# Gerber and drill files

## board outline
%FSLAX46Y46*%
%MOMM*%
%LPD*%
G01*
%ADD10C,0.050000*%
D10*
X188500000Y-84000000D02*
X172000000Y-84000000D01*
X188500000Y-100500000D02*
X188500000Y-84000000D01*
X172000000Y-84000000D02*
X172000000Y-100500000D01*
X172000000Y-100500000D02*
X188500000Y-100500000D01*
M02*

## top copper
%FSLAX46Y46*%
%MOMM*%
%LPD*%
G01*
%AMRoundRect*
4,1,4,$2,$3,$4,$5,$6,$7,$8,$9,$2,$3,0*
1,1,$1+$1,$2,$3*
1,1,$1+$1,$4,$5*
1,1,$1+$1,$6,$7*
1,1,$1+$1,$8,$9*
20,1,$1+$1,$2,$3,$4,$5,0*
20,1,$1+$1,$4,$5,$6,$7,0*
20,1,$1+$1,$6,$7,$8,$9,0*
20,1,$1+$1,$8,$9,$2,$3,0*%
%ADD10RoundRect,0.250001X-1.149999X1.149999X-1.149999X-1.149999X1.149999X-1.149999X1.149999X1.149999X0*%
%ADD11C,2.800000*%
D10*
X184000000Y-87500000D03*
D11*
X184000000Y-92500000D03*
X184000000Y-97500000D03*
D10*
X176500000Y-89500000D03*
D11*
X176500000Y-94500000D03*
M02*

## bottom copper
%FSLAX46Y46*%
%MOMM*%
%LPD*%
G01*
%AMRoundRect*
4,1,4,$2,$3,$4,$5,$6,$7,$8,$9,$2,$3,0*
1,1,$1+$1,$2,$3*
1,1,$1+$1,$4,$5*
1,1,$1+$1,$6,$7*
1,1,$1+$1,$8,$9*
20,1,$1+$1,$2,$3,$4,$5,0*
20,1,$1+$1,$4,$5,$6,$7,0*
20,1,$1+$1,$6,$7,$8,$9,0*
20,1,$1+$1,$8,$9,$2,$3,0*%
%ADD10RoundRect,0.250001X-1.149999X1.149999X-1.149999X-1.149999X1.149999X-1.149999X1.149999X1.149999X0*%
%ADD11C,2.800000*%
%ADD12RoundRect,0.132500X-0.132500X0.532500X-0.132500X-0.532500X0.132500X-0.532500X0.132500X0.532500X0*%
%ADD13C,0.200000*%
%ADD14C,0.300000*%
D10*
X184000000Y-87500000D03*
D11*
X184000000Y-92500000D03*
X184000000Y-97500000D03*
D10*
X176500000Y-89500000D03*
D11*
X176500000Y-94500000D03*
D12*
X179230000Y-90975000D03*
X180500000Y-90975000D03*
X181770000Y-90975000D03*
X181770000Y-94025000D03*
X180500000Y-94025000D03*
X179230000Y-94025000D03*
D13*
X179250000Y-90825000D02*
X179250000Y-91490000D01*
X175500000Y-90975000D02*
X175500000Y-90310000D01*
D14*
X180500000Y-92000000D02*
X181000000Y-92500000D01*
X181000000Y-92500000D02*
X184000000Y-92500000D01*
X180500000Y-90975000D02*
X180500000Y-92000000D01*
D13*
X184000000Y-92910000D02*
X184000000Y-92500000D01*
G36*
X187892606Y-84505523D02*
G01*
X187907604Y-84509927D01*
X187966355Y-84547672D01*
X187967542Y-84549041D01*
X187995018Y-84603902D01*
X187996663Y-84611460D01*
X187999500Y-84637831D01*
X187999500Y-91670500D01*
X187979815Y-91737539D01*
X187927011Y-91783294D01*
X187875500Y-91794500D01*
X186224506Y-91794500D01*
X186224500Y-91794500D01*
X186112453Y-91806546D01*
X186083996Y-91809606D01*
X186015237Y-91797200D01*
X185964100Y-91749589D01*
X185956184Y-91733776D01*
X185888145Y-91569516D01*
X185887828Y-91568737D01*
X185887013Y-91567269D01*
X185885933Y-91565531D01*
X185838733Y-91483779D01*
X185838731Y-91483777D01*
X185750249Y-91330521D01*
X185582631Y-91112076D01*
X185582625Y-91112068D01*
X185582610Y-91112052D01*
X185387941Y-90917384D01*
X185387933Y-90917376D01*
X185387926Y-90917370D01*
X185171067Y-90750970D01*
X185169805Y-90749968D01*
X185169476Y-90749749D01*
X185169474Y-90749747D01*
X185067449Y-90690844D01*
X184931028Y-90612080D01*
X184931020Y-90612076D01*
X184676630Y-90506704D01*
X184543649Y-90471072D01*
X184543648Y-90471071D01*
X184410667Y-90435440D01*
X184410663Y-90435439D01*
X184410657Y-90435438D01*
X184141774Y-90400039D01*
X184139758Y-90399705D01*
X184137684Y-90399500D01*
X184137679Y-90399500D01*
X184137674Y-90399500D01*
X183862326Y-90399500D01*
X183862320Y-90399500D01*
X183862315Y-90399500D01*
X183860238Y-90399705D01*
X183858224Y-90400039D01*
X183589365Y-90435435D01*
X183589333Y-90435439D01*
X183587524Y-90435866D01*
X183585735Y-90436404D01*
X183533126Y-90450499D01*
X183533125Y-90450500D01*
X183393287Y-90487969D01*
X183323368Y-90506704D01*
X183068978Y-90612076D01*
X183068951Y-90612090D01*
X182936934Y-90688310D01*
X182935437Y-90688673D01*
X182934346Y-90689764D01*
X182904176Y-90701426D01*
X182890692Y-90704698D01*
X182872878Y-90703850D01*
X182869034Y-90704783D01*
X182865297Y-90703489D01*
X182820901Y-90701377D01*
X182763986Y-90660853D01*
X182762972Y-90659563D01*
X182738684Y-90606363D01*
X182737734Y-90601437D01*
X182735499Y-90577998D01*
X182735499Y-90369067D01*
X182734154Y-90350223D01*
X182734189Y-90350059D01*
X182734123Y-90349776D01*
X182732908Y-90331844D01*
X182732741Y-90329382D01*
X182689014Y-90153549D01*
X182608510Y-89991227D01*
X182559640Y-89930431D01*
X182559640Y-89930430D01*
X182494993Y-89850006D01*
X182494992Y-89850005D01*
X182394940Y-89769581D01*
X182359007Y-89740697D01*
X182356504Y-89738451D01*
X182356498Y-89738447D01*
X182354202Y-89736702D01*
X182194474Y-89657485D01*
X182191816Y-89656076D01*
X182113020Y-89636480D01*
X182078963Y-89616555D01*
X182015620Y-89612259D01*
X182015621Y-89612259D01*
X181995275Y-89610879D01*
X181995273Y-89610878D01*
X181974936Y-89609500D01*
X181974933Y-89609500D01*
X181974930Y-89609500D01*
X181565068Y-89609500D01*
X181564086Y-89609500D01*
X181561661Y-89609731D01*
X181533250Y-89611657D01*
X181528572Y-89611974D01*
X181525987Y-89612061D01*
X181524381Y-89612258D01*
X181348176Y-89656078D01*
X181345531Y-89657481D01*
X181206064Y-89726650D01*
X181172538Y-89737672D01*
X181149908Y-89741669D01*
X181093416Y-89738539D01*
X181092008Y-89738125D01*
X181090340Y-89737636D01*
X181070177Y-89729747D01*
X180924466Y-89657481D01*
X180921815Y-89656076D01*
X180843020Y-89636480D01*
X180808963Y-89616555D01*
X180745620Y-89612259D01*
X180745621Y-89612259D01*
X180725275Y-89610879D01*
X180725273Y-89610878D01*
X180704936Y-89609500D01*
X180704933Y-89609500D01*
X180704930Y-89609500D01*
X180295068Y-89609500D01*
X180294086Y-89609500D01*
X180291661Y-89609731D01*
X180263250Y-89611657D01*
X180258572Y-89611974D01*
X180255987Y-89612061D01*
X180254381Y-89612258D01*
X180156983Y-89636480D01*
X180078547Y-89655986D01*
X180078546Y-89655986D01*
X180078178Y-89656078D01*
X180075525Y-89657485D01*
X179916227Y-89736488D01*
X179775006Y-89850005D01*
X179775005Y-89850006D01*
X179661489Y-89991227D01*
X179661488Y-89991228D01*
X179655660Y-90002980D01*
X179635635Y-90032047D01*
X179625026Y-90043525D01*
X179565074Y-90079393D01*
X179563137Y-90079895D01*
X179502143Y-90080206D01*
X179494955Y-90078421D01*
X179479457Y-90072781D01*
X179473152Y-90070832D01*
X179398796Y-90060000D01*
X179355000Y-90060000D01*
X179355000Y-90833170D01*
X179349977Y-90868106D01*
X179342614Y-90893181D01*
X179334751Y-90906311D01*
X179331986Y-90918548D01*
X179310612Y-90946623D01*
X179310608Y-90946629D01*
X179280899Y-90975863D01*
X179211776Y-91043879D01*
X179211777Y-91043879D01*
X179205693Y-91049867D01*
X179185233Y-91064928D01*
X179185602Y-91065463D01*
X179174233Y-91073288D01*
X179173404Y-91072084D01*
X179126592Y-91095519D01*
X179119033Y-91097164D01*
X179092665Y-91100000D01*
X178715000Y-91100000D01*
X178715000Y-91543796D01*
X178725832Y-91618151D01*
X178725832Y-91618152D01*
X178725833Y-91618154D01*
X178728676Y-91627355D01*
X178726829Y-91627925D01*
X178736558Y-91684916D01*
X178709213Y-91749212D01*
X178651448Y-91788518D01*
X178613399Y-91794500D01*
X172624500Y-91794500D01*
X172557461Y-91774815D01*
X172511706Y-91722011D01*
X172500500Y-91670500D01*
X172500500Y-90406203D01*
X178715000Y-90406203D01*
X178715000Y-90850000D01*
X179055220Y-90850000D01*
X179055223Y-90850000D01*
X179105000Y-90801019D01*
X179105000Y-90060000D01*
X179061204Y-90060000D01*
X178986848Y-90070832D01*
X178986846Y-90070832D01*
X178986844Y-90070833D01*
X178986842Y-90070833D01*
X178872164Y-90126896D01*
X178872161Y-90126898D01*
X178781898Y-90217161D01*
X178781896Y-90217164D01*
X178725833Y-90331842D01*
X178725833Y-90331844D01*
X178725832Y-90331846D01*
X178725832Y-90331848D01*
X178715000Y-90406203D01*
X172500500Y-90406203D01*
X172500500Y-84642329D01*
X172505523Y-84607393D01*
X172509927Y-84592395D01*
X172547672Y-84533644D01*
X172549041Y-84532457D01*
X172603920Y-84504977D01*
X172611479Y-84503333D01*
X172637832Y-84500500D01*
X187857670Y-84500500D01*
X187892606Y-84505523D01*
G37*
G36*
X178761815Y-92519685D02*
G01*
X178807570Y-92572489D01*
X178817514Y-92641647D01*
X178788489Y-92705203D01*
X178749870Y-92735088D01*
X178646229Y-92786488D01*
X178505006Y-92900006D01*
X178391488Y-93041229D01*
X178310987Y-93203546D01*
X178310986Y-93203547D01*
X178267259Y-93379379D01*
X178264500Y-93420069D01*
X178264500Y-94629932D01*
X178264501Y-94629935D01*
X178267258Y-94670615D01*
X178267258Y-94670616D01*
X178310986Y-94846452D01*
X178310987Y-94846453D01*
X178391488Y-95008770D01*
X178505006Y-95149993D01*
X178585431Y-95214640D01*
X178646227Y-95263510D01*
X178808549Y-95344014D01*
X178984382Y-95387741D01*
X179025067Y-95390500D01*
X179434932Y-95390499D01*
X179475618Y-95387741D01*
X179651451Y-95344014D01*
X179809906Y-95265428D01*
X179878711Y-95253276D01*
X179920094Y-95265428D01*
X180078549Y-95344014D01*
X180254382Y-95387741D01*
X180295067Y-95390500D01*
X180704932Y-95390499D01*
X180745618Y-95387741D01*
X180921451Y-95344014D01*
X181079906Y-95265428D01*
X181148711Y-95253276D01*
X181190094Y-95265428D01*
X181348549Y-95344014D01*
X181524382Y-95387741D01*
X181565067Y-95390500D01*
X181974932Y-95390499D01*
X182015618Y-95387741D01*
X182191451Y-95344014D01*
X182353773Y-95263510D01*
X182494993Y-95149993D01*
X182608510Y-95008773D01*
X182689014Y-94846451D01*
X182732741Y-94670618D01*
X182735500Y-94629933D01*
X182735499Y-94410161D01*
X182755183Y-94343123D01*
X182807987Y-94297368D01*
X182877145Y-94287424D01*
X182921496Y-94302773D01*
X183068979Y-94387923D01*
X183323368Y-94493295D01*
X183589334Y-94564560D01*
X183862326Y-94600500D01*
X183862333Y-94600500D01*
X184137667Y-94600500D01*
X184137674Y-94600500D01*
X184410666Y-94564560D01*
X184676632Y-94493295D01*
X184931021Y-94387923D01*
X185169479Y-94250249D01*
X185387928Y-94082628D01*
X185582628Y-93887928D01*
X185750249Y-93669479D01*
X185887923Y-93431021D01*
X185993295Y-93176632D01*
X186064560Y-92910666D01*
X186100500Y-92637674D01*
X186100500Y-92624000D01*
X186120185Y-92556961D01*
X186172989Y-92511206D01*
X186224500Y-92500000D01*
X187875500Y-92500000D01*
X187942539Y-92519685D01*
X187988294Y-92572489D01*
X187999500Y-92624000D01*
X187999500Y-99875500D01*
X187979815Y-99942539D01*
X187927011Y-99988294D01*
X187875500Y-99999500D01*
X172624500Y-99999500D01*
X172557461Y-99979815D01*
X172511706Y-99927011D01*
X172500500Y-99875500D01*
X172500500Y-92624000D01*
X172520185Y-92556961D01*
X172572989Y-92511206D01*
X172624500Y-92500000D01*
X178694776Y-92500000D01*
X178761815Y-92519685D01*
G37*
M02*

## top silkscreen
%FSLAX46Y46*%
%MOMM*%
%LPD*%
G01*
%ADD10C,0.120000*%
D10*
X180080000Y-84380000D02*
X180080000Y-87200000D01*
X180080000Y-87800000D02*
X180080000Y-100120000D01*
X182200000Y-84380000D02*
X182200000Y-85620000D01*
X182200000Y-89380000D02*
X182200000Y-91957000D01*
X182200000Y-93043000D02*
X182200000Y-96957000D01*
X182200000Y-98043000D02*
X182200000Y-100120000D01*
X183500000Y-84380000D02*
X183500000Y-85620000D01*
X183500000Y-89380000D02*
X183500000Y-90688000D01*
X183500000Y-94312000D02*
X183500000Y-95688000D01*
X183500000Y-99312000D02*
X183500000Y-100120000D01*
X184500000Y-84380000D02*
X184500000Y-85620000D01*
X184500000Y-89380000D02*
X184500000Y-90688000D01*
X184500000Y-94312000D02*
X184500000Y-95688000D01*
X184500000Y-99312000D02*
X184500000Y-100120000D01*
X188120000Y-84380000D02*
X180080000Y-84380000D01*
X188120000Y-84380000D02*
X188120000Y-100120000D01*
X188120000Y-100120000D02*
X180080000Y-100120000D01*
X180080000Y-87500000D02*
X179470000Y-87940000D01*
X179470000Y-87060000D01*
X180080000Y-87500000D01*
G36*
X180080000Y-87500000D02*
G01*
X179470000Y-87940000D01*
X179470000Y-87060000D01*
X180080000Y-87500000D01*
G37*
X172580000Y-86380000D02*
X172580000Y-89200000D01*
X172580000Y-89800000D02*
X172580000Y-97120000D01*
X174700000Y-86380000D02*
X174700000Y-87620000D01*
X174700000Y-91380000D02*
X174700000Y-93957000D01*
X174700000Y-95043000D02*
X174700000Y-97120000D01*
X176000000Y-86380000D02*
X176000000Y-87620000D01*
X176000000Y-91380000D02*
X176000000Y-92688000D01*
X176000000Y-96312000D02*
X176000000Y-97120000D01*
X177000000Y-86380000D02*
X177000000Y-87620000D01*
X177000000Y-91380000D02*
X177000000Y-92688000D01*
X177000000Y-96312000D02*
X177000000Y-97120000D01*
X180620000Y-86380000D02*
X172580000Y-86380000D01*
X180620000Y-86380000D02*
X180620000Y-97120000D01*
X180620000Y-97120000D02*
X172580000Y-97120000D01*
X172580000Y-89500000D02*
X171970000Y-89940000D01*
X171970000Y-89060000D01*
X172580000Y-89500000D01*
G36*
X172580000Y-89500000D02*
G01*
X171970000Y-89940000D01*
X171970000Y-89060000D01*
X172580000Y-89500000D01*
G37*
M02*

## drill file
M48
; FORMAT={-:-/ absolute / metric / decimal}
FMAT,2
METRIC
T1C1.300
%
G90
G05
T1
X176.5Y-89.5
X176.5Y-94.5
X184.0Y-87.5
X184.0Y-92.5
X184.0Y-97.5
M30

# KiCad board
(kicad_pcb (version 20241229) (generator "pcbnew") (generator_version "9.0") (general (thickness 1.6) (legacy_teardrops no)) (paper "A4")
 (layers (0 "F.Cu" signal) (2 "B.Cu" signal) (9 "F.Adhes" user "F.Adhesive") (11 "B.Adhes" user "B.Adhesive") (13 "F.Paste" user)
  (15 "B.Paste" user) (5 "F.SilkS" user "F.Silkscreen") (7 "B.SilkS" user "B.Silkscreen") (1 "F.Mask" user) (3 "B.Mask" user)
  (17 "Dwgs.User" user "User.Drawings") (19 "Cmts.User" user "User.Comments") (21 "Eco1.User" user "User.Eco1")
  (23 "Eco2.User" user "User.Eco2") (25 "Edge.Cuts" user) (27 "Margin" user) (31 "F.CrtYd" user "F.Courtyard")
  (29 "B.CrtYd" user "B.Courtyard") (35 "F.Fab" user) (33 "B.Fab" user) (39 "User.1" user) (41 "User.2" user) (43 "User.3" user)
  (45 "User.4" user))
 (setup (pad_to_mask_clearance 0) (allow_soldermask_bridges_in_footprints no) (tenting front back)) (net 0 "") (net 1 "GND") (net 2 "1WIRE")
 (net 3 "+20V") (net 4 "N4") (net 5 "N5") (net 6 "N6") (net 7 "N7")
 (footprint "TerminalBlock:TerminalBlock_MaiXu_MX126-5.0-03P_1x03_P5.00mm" (layer "F.Cu") (at 184 87.5 -90)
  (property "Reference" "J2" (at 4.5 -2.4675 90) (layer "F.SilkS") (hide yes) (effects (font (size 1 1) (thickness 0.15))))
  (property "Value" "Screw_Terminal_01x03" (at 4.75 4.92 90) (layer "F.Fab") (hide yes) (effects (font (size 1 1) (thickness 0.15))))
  (fp_line (start -3.12 3.92) (end -0.3 3.92) (stroke (width 0.12) (type solid)) (layer "F.SilkS"))
  (fp_line (start 0.3 3.92) (end 12.62 3.92) (stroke (width 0.12) (type solid)) (layer "F.SilkS"))
  (fp_line (start -3.12 1.8) (end -1.88 1.8) (stroke (width 0.12) (type solid)) (layer "F.SilkS"))
  (fp_line (start 1.88 1.8) (end 4.457 1.8) (stroke (width 0.12) (type solid)) (layer "F.SilkS"))
  (fp_line (start 5.543 1.8) (end 9.457 1.8) (stroke (width 0.12) (type solid)) (layer "F.SilkS"))
  (fp_line (start 10.543 1.8) (end 12.62 1.8) (stroke (width 0.12) (type solid)) (layer "F.SilkS"))
  (fp_line (start -3.12 0.5) (end -1.88 0.5) (stroke (width 0.12) (type solid)) (layer "F.SilkS"))
  (fp_line (start 1.88 0.5) (end 3.188 0.5) (stroke (width 0.12) (type solid)) (layer "F.SilkS"))
  (fp_line (start 6.812 0.5) (end 8.188 0.5) (stroke (width 0.12) (type solid)) (layer "F.SilkS"))
  (fp_line (start 11.812 0.5) (end 12.62 0.5) (stroke (width 0.12) (type solid)) (layer "F.SilkS"))
  (fp_line (start -3.12 -0.5) (end -1.88 -0.5) (stroke (width 0.12) (type solid)) (layer "F.SilkS"))
  (fp_line (start 1.88 -0.5) (end 3.188 -0.5) (stroke (width 0.12) (type solid)) (layer "F.SilkS"))
  (fp_line (start 6.812 -0.5) (end 8.188 -0.5) (stroke (width 0.12) (type solid)) (layer "F.SilkS"))
  (fp_line (start 11.812 -0.5) (end 12.62 -0.5) (stroke (width 0.12) (type solid)) (layer "F.SilkS"))
  (fp_line (start -3.12 -4.12) (end -3.12 3.92) (stroke (width 0.12) (type solid)) (layer "F.SilkS"))
  (fp_line (start -3.12 -4.12) (end 12.62 -4.12) (stroke (width 0.12) (type solid)) (layer "F.SilkS"))
  (fp_line (start 12.62 -4.12) (end 12.62 3.92) (stroke (width 0.12) (type solid)) (layer "F.SilkS"))
  (fp_poly (pts (xy 0 3.92) (xy 0.44 4.53) (xy -0.44 4.53)) (stroke (width 0.12) (type solid)) (fill yes) (layer "F.SilkS"))
  (pad "1" thru_hole roundrect (at 0 0 270) (size 2.8 2.8) (drill 1.3) (layers "*.Cu" "*.Mask") (remove_unused_layers no)
   (roundrect_rratio 0.089286) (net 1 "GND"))
  (pad "2" thru_hole circle (at 5 0 270) (size 2.8 2.8) (drill 1.3) (layers "*.Cu" "*.Mask") (remove_unused_layers no) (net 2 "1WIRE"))
  (pad "3" thru_hole circle (at 10 0 270) (size 2.8 2.8) (drill 1.3) (layers "*.Cu" "*.Mask") (remove_unused_layers no) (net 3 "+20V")))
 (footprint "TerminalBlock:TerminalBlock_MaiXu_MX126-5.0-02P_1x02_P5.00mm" (layer "F.Cu") (at 176.5 89.5 -90)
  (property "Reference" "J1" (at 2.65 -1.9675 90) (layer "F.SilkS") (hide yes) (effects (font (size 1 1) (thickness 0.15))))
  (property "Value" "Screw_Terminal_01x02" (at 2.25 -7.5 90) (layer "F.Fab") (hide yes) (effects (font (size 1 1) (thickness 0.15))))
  (fp_line (start -3.12 3.92) (end -0.3 3.92) (stroke (width 0.12) (type solid)) (layer "F.SilkS"))
  (fp_line (start 0.3 3.92) (end 7.62 3.92) (stroke (width 0.12) (type solid)) (layer "F.SilkS"))
  (fp_line (start -3.12 1.8) (end -1.88 1.8) (stroke (width 0.12) (type solid)) (layer "F.SilkS"))
  (fp_line (start 1.88 1.8) (end 4.457 1.8) (stroke (width 0.12) (type solid)) (layer "F.SilkS"))
  (fp_line (start 5.543 1.8) (end 7.62 1.8) (stroke (width 0.12) (type solid)) (layer "F.SilkS"))
  (fp_line (start -3.12 0.5) (end -1.88 0.5) (stroke (width 0.12) (type solid)) (layer "F.SilkS"))
  (fp_line (start 1.88 0.5) (end 3.188 0.5) (stroke (width 0.12) (type solid)) (layer "F.SilkS"))
  (fp_line (start 6.812 0.5) (end 7.62 0.5) (stroke (width 0.12) (type solid)) (layer "F.SilkS"))
  (fp_line (start -3.12 -0.5) (end -1.88 -0.5) (stroke (width 0.12) (type solid)) (layer "F.SilkS"))
  (fp_line (start 1.88 -0.5) (end 3.188 -0.5) (stroke (width 0.12) (type solid)) (layer "F.SilkS"))
  (fp_line (start 6.812 -0.5) (end 7.62 -0.5) (stroke (width 0.12) (type solid)) (layer "F.SilkS"))
  (fp_line (start -3.12 -4.12) (end -3.12 3.92) (stroke (width 0.12) (type solid)) (layer "F.SilkS"))
  (fp_line (start -3.12 -4.12) (end 7.62 -4.12) (stroke (width 0.12) (type solid)) (layer "F.SilkS"))
  (fp_line (start 7.62 -4.12) (end 7.62 3.92) (stroke (width 0.12) (type solid)) (layer "F.SilkS"))
  (fp_poly (pts (xy 0 3.92) (xy 0.44 4.53) (xy -0.44 4.53)) (stroke (width 0.12) (type solid)) (fill yes) (layer "F.SilkS"))
  (pad "1" thru_hole roundrect (at 0 0 270) (size 2.8 2.8) (drill 1.3) (layers "*.Cu" "*.Mask") (remove_unused_layers no)
   (roundrect_rratio 0.089286) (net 1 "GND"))
  (pad "2" thru_hole circle (at 5 0 270) (size 2.8 2.8) (drill 1.3) (layers "*.Cu" "*.Mask") (remove_unused_layers no) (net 3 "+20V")))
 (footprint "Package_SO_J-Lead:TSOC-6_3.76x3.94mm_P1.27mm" (layer "B.Cu") (at 180.5 92.5 -90)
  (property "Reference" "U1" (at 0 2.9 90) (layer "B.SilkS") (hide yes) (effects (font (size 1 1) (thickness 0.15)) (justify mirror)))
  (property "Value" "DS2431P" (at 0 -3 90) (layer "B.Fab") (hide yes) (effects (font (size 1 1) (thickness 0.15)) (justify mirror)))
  (pad "1" smd roundrect (at -1.525 1.27 270) (size 1.33 0.53) (layers "B.Cu" "B.Mask" "B.Paste") (roundrect_rratio 0.25) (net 1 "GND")
   (zone_connect 1) (thermal_bridge_width 0.203) (thermal_gap 0.25))
  (pad "2" smd roundrect (at -1.525 0 270) (size 1.33 0.53) (layers "B.Cu" "B.Mask" "B.Paste") (roundrect_rratio 0.25) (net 2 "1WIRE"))
  (pad "3" smd roundrect (at -1.525 -1.27 270) (size 1.33 0.53) (layers "B.Cu" "B.Mask" "B.Paste") (roundrect_rratio 0.25) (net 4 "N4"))
  (pad "4" smd roundrect (at 1.525 -1.27 270) (size 1.33 0.53) (layers "B.Cu" "B.Mask" "B.Paste") (roundrect_rratio 0.25) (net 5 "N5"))
  (pad "5" smd roundrect (at 1.525 0 270) (size 1.33 0.53) (layers "B.Cu" "B.Mask" "B.Paste") (roundrect_rratio 0.25) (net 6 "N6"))
  (pad "6" smd roundrect (at 1.525 1.27 270) (size 1.33 0.53) (layers "B.Cu" "B.Mask" "B.Paste") (roundrect_rratio 0.25) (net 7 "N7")))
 (gr_line (start 188.5 84) (end 172 84) (stroke (width 0.05) (type default)) (layer "Edge.Cuts"))
 (gr_line (start 188.5 100.5) (end 188.5 84) (stroke (width 0.05) (type default)) (layer "Edge.Cuts"))
 (gr_line (start 172 84) (end 172 100.5) (stroke (width 0.05) (type default)) (layer "Edge.Cuts"))
 (gr_line (start 172 100.5) (end 188.5 100.5) (stroke (width 0.05) (type default)) (layer "Edge.Cuts"))
 (segment (start 179.25 90.825) (end 179.25 91.49) (width 0.2) (layer "B.Cu") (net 1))
 (segment (start 175.5 90.975) (end 175.5 90.31) (width 0.2) (layer "B.Cu") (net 1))
 (segment (start 180.5 92) (end 181 92.5) (width 0.3) (layer "B.Cu") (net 2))
 (segment (start 181 92.5) (end 184 92.5) (width 0.3) (layer "B.Cu") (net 2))
 (segment (start 180.5 90.975) (end 180.5 92) (width 0.3) (layer "B.Cu") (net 2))
 (segment (start 184 92.91) (end 184 92.5) (width 0.2) (layer "B.Cu") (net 2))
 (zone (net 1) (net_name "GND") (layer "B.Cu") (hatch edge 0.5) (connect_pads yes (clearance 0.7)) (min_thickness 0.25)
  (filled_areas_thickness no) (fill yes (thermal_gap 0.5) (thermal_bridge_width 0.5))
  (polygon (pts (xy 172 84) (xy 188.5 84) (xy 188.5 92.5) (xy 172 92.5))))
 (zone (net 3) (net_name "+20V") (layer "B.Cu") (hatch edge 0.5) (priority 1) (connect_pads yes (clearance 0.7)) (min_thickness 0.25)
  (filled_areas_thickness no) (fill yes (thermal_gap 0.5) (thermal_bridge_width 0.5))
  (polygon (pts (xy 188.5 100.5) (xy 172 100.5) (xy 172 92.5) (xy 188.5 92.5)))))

